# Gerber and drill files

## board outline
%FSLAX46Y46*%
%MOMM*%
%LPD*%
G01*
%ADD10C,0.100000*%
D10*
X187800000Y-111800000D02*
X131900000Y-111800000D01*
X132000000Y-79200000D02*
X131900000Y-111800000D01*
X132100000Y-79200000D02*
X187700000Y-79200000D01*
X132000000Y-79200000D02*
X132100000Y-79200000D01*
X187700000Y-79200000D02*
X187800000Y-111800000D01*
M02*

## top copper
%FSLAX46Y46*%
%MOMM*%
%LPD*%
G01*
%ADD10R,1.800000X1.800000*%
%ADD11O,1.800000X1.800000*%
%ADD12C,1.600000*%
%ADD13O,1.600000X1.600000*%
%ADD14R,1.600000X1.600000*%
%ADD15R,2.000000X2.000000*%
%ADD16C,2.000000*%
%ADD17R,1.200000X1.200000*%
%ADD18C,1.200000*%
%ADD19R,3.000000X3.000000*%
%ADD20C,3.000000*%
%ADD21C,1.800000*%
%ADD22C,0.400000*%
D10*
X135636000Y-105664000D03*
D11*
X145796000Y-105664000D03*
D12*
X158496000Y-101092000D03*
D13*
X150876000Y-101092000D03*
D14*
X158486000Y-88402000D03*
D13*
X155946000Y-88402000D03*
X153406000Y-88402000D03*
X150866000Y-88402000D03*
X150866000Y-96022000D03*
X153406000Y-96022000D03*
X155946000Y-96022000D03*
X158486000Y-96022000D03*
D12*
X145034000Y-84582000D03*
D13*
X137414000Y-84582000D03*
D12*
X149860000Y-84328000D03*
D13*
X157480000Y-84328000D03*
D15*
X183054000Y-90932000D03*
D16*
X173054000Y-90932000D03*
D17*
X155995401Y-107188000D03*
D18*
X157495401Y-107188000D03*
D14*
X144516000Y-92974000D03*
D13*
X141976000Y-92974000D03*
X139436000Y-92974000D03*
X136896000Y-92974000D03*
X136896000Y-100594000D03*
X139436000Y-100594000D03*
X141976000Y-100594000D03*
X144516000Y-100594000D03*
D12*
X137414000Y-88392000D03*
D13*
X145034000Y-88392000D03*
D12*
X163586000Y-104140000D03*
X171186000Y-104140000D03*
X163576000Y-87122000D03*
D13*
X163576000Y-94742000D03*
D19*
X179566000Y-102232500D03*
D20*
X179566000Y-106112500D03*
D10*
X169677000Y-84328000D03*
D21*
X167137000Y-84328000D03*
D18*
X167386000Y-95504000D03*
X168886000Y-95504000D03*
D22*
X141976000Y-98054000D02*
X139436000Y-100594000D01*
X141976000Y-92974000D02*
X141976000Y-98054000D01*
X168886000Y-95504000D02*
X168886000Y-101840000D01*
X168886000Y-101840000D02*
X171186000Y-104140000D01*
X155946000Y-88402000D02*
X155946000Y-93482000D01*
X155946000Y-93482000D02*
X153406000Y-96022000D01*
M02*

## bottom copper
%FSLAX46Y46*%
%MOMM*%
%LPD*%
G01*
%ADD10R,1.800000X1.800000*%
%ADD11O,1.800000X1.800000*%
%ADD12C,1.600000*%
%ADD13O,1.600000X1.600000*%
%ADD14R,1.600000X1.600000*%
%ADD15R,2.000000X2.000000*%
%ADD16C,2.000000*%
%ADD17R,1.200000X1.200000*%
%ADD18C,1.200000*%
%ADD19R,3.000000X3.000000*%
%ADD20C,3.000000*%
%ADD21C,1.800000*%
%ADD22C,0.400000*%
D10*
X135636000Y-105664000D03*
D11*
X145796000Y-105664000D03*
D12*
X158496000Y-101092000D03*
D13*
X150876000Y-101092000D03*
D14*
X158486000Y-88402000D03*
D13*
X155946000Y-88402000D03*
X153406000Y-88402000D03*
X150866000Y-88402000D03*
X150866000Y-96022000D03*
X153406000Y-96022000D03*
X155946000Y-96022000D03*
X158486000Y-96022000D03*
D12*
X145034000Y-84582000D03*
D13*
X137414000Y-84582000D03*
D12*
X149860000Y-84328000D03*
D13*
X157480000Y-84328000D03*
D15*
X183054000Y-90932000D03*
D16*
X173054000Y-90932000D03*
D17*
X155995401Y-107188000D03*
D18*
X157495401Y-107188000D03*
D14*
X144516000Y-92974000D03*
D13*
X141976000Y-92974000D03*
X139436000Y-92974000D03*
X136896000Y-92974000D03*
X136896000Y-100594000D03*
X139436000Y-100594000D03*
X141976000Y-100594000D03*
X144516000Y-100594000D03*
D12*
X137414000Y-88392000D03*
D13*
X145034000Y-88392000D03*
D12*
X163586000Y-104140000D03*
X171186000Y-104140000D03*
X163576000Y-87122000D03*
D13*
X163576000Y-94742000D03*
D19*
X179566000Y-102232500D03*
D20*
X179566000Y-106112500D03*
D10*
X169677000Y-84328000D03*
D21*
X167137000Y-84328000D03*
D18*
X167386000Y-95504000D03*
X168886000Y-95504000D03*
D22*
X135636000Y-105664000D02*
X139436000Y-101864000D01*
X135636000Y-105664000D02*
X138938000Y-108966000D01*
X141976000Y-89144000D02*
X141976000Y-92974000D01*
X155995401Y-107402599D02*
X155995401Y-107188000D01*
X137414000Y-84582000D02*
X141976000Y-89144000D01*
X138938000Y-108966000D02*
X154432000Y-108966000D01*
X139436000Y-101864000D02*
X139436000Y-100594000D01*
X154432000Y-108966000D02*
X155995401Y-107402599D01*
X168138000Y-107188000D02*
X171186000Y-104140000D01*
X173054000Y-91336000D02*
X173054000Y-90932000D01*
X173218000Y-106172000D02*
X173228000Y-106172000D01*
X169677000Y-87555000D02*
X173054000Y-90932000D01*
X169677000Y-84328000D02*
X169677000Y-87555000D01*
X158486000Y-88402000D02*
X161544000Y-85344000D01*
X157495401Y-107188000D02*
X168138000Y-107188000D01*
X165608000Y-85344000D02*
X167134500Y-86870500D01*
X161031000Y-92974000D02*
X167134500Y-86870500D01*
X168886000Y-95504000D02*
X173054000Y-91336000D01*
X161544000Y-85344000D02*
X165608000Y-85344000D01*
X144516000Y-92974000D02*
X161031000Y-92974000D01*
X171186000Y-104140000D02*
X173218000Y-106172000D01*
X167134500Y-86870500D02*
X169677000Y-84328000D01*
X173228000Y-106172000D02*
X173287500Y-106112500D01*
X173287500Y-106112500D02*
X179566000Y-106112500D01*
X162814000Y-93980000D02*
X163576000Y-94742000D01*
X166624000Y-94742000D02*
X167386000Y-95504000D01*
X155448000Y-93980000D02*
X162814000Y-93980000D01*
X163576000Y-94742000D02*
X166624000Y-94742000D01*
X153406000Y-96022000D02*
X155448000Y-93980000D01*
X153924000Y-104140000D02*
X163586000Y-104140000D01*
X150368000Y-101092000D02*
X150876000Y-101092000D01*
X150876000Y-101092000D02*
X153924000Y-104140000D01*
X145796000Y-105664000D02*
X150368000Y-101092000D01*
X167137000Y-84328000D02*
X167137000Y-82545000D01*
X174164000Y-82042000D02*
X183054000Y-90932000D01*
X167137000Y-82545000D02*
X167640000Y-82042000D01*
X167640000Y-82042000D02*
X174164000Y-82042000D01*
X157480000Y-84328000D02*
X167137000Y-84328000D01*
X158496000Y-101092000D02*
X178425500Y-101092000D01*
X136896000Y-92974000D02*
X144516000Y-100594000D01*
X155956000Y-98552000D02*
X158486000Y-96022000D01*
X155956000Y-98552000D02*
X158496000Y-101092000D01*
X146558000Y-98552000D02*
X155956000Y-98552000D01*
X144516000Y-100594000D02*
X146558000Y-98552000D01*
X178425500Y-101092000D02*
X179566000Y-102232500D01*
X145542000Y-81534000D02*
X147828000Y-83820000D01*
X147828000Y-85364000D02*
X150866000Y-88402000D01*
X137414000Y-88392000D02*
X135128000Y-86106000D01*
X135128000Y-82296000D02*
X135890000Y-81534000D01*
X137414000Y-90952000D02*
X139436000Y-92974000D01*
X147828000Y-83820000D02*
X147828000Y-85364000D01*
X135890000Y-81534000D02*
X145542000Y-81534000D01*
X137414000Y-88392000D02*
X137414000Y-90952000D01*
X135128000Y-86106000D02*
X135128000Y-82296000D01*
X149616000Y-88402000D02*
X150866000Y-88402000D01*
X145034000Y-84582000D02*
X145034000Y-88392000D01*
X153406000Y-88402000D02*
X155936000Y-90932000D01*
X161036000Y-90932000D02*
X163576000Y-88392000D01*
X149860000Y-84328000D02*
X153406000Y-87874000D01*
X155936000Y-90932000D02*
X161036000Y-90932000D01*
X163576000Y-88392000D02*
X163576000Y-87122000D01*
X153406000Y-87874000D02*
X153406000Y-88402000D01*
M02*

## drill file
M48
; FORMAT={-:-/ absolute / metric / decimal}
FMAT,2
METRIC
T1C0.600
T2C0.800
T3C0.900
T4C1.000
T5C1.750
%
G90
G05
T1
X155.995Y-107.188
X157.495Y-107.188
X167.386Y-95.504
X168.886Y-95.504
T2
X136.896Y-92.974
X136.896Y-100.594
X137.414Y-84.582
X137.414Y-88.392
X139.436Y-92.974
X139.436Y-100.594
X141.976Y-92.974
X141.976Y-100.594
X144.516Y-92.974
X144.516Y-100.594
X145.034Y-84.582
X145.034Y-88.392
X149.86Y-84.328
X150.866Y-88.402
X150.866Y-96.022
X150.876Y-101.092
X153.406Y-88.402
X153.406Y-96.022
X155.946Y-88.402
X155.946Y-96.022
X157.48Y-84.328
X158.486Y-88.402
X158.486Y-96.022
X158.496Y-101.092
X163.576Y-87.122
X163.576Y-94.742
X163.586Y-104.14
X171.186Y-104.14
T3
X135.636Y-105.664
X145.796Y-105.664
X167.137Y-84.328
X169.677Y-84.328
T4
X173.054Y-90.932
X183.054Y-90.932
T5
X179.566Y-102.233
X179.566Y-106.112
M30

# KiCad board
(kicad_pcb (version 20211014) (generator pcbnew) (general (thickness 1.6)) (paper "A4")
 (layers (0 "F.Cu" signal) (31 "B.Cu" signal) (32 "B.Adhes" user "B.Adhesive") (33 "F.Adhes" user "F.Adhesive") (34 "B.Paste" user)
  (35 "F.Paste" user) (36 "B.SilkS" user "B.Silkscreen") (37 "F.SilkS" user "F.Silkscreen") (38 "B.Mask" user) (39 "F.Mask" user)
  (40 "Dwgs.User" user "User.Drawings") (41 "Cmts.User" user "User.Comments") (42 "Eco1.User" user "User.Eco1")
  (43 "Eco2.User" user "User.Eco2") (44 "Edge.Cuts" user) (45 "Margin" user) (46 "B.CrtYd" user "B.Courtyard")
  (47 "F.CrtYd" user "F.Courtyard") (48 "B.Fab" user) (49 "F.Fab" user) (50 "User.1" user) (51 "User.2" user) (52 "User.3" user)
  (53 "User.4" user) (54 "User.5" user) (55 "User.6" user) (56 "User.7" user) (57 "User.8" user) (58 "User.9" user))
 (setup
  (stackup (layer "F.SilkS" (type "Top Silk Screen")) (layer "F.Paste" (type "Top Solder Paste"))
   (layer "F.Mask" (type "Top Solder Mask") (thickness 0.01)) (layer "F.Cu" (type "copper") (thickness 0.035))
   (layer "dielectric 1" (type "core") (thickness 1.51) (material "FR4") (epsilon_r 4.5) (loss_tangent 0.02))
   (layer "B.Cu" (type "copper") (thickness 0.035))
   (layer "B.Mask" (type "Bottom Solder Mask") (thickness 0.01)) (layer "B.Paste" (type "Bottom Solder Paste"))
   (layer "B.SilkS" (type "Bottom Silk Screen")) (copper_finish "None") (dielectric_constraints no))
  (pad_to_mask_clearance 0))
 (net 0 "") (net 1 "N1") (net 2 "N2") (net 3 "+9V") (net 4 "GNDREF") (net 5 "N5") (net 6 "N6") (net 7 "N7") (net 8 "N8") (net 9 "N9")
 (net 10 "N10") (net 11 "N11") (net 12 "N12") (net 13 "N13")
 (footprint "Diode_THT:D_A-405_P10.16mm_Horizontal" (layer "F.Cu") (at 135.636 105.664)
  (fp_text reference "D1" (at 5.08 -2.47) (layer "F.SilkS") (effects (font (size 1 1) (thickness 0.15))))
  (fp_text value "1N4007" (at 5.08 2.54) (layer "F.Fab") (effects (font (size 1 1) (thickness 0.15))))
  (pad "1" thru_hole rect locked (at 0 0) (size 1.8 1.8) (drill 0.9) (layers *.Cu *.Mask) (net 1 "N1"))
  (pad "2" thru_hole oval locked (at 10.16 0) (size 1.8 1.8) (drill 0.9) (layers *.Cu *.Mask) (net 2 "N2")))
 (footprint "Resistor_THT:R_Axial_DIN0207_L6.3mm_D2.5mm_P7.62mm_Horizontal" (layer "F.Cu") (at 158.496 101.092 180)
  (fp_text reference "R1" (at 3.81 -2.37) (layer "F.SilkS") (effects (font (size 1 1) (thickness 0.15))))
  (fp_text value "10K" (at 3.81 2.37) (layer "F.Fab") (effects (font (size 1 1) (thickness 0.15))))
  (pad "1" thru_hole circle locked (at 0 0 180) (size 1.6 1.6) (drill 0.8) (layers *.Cu *.Mask) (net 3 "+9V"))
  (pad "2" thru_hole oval locked (at 7.62 0 180) (size 1.6 1.6) (drill 0.8) (layers *.Cu *.Mask) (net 2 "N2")))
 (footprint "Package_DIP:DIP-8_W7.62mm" (layer "F.Cu") (at 158.486 88.402 -90)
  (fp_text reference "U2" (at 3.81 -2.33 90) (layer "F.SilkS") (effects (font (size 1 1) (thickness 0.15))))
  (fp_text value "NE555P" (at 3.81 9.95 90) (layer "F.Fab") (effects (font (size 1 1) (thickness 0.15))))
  (pad "1" thru_hole rect locked (at 0 0 270) (size 1.6 1.6) (drill 0.8) (layers *.Cu *.Mask) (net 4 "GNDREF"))
  (pad "2" thru_hole oval locked (at 0 2.54 270) (size 1.6 1.6) (drill 0.8) (layers *.Cu *.Mask) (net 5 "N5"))
  (pad "3" thru_hole oval locked (at 0 5.08 270) (size 1.6 1.6) (drill 0.8) (layers *.Cu *.Mask) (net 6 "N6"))
  (pad "4" thru_hole oval locked (at 0 7.62 270) (size 1.6 1.6) (drill 0.8) (layers *.Cu *.Mask) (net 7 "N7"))
  (pad "5" thru_hole oval locked (at 7.62 7.62 270) (size 1.6 1.6) (drill 0.8) (layers *.Cu *.Mask) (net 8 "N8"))
  (pad "6" thru_hole oval locked (at 7.62 5.08 270) (size 1.6 1.6) (drill 0.8) (layers *.Cu *.Mask) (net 5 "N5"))
  (pad "7" thru_hole oval locked (at 7.62 2.54 270) (size 1.6 1.6) (drill 0.8) (layers *.Cu *.Mask) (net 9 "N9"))
  (pad "8" thru_hole oval locked (at 7.62 0 270) (size 1.6 1.6) (drill 0.8) (layers *.Cu *.Mask) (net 3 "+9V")))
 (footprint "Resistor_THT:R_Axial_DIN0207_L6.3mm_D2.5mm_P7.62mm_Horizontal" (layer "F.Cu") (at 145.034 84.582 180)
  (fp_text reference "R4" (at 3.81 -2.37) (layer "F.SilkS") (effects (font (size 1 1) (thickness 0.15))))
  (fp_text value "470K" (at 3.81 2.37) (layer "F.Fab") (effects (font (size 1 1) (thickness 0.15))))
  (pad "1" thru_hole circle locked (at 0 0 180) (size 1.6 1.6) (drill 0.8) (layers *.Cu *.Mask) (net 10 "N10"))
  (pad "2" thru_hole oval locked (at 7.62 0 180) (size 1.6 1.6) (drill 0.8) (layers *.Cu *.Mask) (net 1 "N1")))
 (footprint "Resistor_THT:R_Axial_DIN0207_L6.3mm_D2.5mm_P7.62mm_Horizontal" (layer "F.Cu") (at 149.86 84.328)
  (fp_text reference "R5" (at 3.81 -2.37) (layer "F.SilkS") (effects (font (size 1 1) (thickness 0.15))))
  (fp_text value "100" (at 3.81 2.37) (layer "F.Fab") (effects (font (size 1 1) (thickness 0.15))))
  (pad "1" thru_hole circle locked (at 0 0) (size 1.6 1.6) (drill 0.8) (layers *.Cu *.Mask) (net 6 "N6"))
  (pad "2" thru_hole oval locked (at 7.62 0) (size 1.6 1.6) (drill 0.8) (layers *.Cu *.Mask) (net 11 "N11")))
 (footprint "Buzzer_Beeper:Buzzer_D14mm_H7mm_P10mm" (layer "F.Cu") (at 183.054 90.932 180)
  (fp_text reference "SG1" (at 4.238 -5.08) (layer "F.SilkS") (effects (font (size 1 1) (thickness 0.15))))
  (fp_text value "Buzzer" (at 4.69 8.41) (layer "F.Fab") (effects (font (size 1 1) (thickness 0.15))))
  (pad "1" thru_hole rect locked (at 0 0 180) (size 2 2) (drill 1) (layers *.Cu *.Mask) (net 11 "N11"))
  (pad "2" thru_hole circle locked (at 10 0 180) (size 2 2) (drill 1) (layers *.Cu *.Mask) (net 4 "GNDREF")))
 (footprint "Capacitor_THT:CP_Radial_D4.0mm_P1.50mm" (layer "F.Cu") (at 155.995401 107.188)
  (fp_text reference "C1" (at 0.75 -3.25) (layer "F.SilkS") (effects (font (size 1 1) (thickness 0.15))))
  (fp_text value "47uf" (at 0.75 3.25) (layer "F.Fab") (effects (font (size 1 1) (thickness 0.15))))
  (pad "1" thru_hole rect locked (at 0 0) (size 1.2 1.2) (drill 0.6) (layers *.Cu *.Mask) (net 1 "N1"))
  (pad "2" thru_hole circle locked (at 1.5 0) (size 1.2 1.2) (drill 0.6) (layers *.Cu *.Mask) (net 4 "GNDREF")))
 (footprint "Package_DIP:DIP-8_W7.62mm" (layer "F.Cu") (at 144.516 92.974 -90)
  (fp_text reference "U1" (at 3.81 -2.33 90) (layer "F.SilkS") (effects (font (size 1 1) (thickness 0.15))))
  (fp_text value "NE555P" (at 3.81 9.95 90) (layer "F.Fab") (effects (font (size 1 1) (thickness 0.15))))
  (pad "1" thru_hole rect locked (at 0 0 270) (size 1.6 1.6) (drill 0.8) (layers *.Cu *.Mask) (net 4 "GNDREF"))
  (pad "2" thru_hole oval locked (at 0 2.54 270) (size 1.6 1.6) (drill 0.8) (layers *.Cu *.Mask) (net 1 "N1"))
  (pad "3" thru_hole oval locked (at 0 5.08 270) (size 1.6 1.6) (drill 0.8) (layers *.Cu *.Mask) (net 7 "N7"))
  (pad "4" thru_hole oval locked (at 0 7.62 270) (size 1.6 1.6) (drill 0.8) (layers *.Cu *.Mask) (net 3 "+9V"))
  (pad "5" thru_hole oval locked (at 7.62 7.62 270) (size 1.6 1.6) (drill 0.8) (layers *.Cu *.Mask) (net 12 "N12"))
  (pad "6" thru_hole oval locked (at 7.62 5.08 270) (size 1.6 1.6) (drill 0.8) (layers *.Cu *.Mask) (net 1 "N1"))
  (pad "7" thru_hole oval locked (at 7.62 2.54 270) (size 1.6 1.6) (drill 0.8) (layers *.Cu *.Mask) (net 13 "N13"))
  (pad "8" thru_hole oval locked (at 7.62 0 270) (size 1.6 1.6) (drill 0.8) (layers *.Cu *.Mask) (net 3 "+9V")))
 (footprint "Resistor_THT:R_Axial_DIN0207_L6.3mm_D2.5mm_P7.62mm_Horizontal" (layer "F.Cu") (at 137.414 88.392)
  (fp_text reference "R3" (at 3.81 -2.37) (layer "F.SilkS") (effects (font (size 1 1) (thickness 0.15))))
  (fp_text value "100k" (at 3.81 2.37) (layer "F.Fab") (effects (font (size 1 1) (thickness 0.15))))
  (pad "1" thru_hole circle locked (at 0 0) (size 1.6 1.6) (drill 0.8) (layers *.Cu *.Mask) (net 7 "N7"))
  (pad "2" thru_hole oval locked (at 7.62 0) (size 1.6 1.6) (drill 0.8) (layers *.Cu *.Mask) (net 10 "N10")))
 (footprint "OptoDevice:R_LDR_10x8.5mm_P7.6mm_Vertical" (layer "F.Cu") (at 163.586 104.14)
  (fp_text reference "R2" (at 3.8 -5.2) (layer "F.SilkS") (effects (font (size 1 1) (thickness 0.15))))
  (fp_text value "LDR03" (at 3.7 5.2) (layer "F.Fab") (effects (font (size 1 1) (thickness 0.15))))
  (pad "1" thru_hole circle locked (at 0 0) (size 1.6 1.6) (drill 0.8) (layers *.Cu *.Mask) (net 2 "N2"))
  (pad "2" thru_hole circle locked (at 7.6 0) (size 1.6 1.6) (drill 0.8) (layers *.Cu *.Mask) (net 4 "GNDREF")))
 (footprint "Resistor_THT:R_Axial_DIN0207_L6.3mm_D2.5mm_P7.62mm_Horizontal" (layer "F.Cu") (at 163.576 87.122 -90)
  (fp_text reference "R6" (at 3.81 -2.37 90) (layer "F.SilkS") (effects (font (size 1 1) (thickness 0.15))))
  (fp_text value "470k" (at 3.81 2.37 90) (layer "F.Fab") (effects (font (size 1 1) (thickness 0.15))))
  (pad "1" thru_hole circle locked (at 0 0 270) (size 1.6 1.6) (drill 0.8) (layers *.Cu *.Mask) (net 6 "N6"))
  (pad "2" thru_hole oval locked (at 7.62 0 270) (size 1.6 1.6) (drill 0.8) (layers *.Cu *.Mask) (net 5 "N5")))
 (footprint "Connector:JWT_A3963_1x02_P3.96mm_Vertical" (layer "F.Cu") (at 179.566 102.2325 -90)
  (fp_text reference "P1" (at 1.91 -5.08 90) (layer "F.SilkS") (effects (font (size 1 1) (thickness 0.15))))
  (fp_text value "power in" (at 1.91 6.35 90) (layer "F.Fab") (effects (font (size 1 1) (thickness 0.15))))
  (pad "1" thru_hole rect locked (at 0 0 270) (size 3 3) (drill 1.75) (layers *.Cu *.Mask) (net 3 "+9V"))
  (pad "2" thru_hole circle locked (at 3.88 0 270) (size 3 3) (drill 1.75) (layers *.Cu *.Mask) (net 4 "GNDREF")))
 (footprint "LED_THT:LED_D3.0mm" (layer "F.Cu") (at 169.677 84.328 180)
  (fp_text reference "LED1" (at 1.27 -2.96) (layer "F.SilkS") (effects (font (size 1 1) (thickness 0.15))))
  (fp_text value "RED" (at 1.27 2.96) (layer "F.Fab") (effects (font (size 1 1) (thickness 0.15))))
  (pad "1" thru_hole rect locked (at 0 0 180) (size 1.8 1.8) (drill 0.9) (layers *.Cu *.Mask) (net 4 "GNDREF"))
  (pad "2" thru_hole circle locked (at 2.54 0 180) (size 1.8 1.8) (drill 0.9) (layers *.Cu *.Mask) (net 11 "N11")))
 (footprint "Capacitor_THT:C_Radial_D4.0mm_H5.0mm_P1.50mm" (layer "F.Cu") (at 167.386 95.504)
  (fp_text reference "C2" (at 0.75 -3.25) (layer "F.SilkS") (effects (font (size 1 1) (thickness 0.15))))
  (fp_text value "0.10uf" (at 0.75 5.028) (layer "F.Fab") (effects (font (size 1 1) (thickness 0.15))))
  (pad "1" thru_hole circle locked (at 0 0) (size 1.2 1.2) (drill 0.6) (layers *.Cu *.Mask) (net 5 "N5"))
  (pad "2" thru_hole circle locked (at 1.5 0) (size 1.2 1.2) (drill 0.6) (layers *.Cu *.Mask) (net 4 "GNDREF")))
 (gr_line (start 187.8 111.8) (end 131.9 111.8) (layer "Edge.Cuts") (width 0.1))
 (gr_line (start 132 79.2) (end 131.9 111.8) (layer "Edge.Cuts") (width 0.1))
 (gr_line (start 132.1 79.2) (end 187.7 79.2) (layer "Edge.Cuts") (width 0.1))
 (gr_line (start 132 79.2) (end 132.1 79.2) (layer "Edge.Cuts") (width 0.1))
 (gr_line (start 187.7 79.2) (end 187.8 111.8) (layer "Edge.Cuts") (width 0.1))
 (segment (start 141.976 98.054) (end 139.436 100.594) (width 0.4) (layer "F.Cu") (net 1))
 (segment (start 141.976 92.974) (end 141.976 98.054) (width 0.4) (layer "F.Cu") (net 1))
 (segment (start 135.636 105.664) (end 139.436 101.864) (width 0.4) (layer "B.Cu") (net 1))
 (segment (start 135.636 105.664) (end 138.938 108.966) (width 0.4) (layer "B.Cu") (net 1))
 (segment (start 141.976 89.144) (end 141.976 92.974) (width 0.4) (layer "B.Cu") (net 1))
 (segment (start 155.995401 107.402599) (end 155.995401 107.188) (width 0.4) (layer "B.Cu") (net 1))
 (segment (start 137.414 84.582) (end 141.976 89.144) (width 0.4) (layer "B.Cu") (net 1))
 (segment (start 138.938 108.966) (end 154.432 108.966) (width 0.4) (layer "B.Cu") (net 1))
 (segment (start 139.436 101.864) (end 139.436 100.594) (width 0.4) (layer "B.Cu") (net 1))
 (segment (start 154.432 108.966) (end 155.995401 107.402599) (width 0.4) (layer "B.Cu") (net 1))
 (segment (start 168.886 95.504) (end 168.886 101.84) (width 0.4) (layer "F.Cu") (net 4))
 (segment (start 168.886 101.84) (end 171.186 104.14) (width 0.4) (layer "F.Cu") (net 4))
 (segment (start 168.138 107.188) (end 171.186 104.14) (width 0.4) (layer "B.Cu") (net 4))
 (segment (start 173.054 91.336) (end 173.054 90.932) (width 0.4) (layer "B.Cu") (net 4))
 (segment (start 173.218 106.172) (end 173.228 106.172) (width 0.4) (layer "B.Cu") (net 4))
 (segment (start 169.677 87.555) (end 173.054 90.932) (width 0.4) (layer "B.Cu") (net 4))
 (segment (start 169.677 84.328) (end 169.677 87.555) (width 0.4) (layer "B.Cu") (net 4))
 (segment (start 158.486 88.402) (end 161.544 85.344) (width 0.4) (layer "B.Cu") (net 4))
 (segment (start 157.495401 107.188) (end 168.138 107.188) (width 0.4) (layer "B.Cu") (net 4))
 (segment (start 165.608 85.344) (end 167.1345 86.8705) (width 0.4) (layer "B.Cu") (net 4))
 (segment (start 161.031 92.974) (end 167.1345 86.8705) (width 0.4) (layer "B.Cu") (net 4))
 (segment (start 168.886 95.504) (end 173.054 91.336) (width 0.4) (layer "B.Cu") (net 4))
 (segment (start 161.544 85.344) (end 165.608 85.344) (width 0.4) (layer "B.Cu") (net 4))
 (segment (start 144.516 92.974) (end 161.031 92.974) (width 0.4) (layer "B.Cu") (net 4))
 (segment (start 171.186 104.14) (end 173.218 106.172) (width 0.4) (layer "B.Cu") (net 4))
 (segment (start 167.1345 86.8705) (end 169.677 84.328) (width 0.4) (layer "B.Cu") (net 4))
 (segment (start 173.228 106.172) (end 173.2875 106.1125) (width 0.4) (layer "B.Cu") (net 4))
 (segment (start 173.2875 106.1125) (end 179.566 106.1125) (width 0.4) (layer "B.Cu") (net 4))
 (segment (start 155.946 88.402) (end 155.946 93.482) (width 0.4) (layer "F.Cu") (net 5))
 (segment (start 155.946 93.482) (end 153.406 96.022) (width 0.4) (layer "F.Cu") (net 5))
 (segment (start 162.814 93.98) (end 163.576 94.742) (width 0.4) (layer "B.Cu") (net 5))
 (segment (start 166.624 94.742) (end 167.386 95.504) (width 0.4) (layer "B.Cu") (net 5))
 (segment (start 155.448 93.98) (end 162.814 93.98) (width 0.4) (layer "B.Cu") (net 5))
 (segment (start 163.576 94.742) (end 166.624 94.742) (width 0.4) (layer "B.Cu") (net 5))
 (segment (start 153.406 96.022) (end 155.448 93.98) (width 0.4) (layer "B.Cu") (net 5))
 (segment (start 153.924 104.14) (end 163.586 104.14) (width 0.4) (layer "B.Cu") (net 2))
 (segment (start 150.368 101.092) (end 150.876 101.092) (width 0.4) (layer "B.Cu") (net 2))
 (segment (start 150.876 101.092) (end 153.924 104.14) (width 0.4) (layer "B.Cu") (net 2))
 (segment (start 145.796 105.664) (end 150.368 101.092) (width 0.4) (layer "B.Cu") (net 2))
 (segment (start 167.137 84.328) (end 167.137 82.545) (width 0.4) (layer "B.Cu") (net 11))
 (segment (start 174.164 82.042) (end 183.054 90.932) (width 0.4) (layer "B.Cu") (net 11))
 (segment (start 167.137 82.545) (end 167.64 82.042) (width 0.4) (layer "B.Cu") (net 11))
 (segment (start 167.64 82.042) (end 174.164 82.042) (width 0.4) (layer "B.Cu") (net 11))
 (segment (start 157.48 84.328) (end 167.137 84.328) (width 0.4) (layer "B.Cu") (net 11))
 (segment (start 158.496 101.092) (end 178.4255 101.092) (width 0.4) (layer "B.Cu") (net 3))
 (segment (start 136.896 92.974) (end 144.516 100.594) (width 0.4) (layer "B.Cu") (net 3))
 (segment (start 155.956 98.552) (end 158.486 96.022) (width 0.4) (layer "B.Cu") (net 3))
 (segment (start 155.956 98.552) (end 158.496 101.092) (width 0.4) (layer "B.Cu") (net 3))
 (segment (start 146.558 98.552) (end 155.956 98.552) (width 0.4) (layer "B.Cu") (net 3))
 (segment (start 144.516 100.594) (end 146.558 98.552) (width 0.4) (layer "B.Cu") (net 3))
 (segment (start 178.4255 101.092) (end 179.566 102.2325) (width 0.4) (layer "B.Cu") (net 3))
 (segment (start 145.542 81.534) (end 147.828 83.82) (width 0.4) (layer "B.Cu") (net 7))
 (segment (start 147.828 85.364) (end 150.866 88.402) (width 0.4) (layer "B.Cu") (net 7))
 (segment (start 137.414 88.392) (end 135.128 86.106) (width 0.4) (layer "B.Cu") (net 7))
 (segment (start 135.128 82.296) (end 135.89 81.534) (width 0.4) (layer "B.Cu") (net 7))
 (segment (start 137.414 90.952) (end 139.436 92.974) (width 0.4) (layer "B.Cu") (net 7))
 (segment (start 147.828 83.82) (end 147.828 85.364) (width 0.4) (layer "B.Cu") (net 7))
 (segment (start 135.89 81.534) (end 145.542 81.534) (width 0.4) (layer "B.Cu") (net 7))
 (segment (start 137.414 88.392) (end 137.414 90.952) (width 0.4) (layer "B.Cu") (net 7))
 (segment (start 135.128 86.106) (end 135.128 82.296) (width 0.4) (layer "B.Cu") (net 7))
 (segment (start 149.616 88.402) (end 150.866 88.402) (width 0.4) (layer "B.Cu") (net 7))
 (segment (start 145.034 84.582) (end 145.034 88.392) (width 0.4) (layer "B.Cu") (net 10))
 (segment (start 153.406 88.402) (end 155.936 90.932) (width 0.4) (layer "B.Cu") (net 6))
 (segment (start 161.036 90.932) (end 163.576 88.392) (width 0.4) (layer "B.Cu") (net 6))
 (segment (start 149.86 84.328) (end 153.406 87.874) (width 0.4) (layer "B.Cu") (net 6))
 (segment (start 155.936 90.932) (end 161.036 90.932) (width 0.4) (layer "B.Cu") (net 6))
 (segment (start 163.576 88.392) (end 163.576 87.122) (width 0.4) (layer "B.Cu") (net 6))
 (segment (start 153.406 87.874) (end 153.406 88.402) (width 0.4) (layer "B.Cu") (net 6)))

